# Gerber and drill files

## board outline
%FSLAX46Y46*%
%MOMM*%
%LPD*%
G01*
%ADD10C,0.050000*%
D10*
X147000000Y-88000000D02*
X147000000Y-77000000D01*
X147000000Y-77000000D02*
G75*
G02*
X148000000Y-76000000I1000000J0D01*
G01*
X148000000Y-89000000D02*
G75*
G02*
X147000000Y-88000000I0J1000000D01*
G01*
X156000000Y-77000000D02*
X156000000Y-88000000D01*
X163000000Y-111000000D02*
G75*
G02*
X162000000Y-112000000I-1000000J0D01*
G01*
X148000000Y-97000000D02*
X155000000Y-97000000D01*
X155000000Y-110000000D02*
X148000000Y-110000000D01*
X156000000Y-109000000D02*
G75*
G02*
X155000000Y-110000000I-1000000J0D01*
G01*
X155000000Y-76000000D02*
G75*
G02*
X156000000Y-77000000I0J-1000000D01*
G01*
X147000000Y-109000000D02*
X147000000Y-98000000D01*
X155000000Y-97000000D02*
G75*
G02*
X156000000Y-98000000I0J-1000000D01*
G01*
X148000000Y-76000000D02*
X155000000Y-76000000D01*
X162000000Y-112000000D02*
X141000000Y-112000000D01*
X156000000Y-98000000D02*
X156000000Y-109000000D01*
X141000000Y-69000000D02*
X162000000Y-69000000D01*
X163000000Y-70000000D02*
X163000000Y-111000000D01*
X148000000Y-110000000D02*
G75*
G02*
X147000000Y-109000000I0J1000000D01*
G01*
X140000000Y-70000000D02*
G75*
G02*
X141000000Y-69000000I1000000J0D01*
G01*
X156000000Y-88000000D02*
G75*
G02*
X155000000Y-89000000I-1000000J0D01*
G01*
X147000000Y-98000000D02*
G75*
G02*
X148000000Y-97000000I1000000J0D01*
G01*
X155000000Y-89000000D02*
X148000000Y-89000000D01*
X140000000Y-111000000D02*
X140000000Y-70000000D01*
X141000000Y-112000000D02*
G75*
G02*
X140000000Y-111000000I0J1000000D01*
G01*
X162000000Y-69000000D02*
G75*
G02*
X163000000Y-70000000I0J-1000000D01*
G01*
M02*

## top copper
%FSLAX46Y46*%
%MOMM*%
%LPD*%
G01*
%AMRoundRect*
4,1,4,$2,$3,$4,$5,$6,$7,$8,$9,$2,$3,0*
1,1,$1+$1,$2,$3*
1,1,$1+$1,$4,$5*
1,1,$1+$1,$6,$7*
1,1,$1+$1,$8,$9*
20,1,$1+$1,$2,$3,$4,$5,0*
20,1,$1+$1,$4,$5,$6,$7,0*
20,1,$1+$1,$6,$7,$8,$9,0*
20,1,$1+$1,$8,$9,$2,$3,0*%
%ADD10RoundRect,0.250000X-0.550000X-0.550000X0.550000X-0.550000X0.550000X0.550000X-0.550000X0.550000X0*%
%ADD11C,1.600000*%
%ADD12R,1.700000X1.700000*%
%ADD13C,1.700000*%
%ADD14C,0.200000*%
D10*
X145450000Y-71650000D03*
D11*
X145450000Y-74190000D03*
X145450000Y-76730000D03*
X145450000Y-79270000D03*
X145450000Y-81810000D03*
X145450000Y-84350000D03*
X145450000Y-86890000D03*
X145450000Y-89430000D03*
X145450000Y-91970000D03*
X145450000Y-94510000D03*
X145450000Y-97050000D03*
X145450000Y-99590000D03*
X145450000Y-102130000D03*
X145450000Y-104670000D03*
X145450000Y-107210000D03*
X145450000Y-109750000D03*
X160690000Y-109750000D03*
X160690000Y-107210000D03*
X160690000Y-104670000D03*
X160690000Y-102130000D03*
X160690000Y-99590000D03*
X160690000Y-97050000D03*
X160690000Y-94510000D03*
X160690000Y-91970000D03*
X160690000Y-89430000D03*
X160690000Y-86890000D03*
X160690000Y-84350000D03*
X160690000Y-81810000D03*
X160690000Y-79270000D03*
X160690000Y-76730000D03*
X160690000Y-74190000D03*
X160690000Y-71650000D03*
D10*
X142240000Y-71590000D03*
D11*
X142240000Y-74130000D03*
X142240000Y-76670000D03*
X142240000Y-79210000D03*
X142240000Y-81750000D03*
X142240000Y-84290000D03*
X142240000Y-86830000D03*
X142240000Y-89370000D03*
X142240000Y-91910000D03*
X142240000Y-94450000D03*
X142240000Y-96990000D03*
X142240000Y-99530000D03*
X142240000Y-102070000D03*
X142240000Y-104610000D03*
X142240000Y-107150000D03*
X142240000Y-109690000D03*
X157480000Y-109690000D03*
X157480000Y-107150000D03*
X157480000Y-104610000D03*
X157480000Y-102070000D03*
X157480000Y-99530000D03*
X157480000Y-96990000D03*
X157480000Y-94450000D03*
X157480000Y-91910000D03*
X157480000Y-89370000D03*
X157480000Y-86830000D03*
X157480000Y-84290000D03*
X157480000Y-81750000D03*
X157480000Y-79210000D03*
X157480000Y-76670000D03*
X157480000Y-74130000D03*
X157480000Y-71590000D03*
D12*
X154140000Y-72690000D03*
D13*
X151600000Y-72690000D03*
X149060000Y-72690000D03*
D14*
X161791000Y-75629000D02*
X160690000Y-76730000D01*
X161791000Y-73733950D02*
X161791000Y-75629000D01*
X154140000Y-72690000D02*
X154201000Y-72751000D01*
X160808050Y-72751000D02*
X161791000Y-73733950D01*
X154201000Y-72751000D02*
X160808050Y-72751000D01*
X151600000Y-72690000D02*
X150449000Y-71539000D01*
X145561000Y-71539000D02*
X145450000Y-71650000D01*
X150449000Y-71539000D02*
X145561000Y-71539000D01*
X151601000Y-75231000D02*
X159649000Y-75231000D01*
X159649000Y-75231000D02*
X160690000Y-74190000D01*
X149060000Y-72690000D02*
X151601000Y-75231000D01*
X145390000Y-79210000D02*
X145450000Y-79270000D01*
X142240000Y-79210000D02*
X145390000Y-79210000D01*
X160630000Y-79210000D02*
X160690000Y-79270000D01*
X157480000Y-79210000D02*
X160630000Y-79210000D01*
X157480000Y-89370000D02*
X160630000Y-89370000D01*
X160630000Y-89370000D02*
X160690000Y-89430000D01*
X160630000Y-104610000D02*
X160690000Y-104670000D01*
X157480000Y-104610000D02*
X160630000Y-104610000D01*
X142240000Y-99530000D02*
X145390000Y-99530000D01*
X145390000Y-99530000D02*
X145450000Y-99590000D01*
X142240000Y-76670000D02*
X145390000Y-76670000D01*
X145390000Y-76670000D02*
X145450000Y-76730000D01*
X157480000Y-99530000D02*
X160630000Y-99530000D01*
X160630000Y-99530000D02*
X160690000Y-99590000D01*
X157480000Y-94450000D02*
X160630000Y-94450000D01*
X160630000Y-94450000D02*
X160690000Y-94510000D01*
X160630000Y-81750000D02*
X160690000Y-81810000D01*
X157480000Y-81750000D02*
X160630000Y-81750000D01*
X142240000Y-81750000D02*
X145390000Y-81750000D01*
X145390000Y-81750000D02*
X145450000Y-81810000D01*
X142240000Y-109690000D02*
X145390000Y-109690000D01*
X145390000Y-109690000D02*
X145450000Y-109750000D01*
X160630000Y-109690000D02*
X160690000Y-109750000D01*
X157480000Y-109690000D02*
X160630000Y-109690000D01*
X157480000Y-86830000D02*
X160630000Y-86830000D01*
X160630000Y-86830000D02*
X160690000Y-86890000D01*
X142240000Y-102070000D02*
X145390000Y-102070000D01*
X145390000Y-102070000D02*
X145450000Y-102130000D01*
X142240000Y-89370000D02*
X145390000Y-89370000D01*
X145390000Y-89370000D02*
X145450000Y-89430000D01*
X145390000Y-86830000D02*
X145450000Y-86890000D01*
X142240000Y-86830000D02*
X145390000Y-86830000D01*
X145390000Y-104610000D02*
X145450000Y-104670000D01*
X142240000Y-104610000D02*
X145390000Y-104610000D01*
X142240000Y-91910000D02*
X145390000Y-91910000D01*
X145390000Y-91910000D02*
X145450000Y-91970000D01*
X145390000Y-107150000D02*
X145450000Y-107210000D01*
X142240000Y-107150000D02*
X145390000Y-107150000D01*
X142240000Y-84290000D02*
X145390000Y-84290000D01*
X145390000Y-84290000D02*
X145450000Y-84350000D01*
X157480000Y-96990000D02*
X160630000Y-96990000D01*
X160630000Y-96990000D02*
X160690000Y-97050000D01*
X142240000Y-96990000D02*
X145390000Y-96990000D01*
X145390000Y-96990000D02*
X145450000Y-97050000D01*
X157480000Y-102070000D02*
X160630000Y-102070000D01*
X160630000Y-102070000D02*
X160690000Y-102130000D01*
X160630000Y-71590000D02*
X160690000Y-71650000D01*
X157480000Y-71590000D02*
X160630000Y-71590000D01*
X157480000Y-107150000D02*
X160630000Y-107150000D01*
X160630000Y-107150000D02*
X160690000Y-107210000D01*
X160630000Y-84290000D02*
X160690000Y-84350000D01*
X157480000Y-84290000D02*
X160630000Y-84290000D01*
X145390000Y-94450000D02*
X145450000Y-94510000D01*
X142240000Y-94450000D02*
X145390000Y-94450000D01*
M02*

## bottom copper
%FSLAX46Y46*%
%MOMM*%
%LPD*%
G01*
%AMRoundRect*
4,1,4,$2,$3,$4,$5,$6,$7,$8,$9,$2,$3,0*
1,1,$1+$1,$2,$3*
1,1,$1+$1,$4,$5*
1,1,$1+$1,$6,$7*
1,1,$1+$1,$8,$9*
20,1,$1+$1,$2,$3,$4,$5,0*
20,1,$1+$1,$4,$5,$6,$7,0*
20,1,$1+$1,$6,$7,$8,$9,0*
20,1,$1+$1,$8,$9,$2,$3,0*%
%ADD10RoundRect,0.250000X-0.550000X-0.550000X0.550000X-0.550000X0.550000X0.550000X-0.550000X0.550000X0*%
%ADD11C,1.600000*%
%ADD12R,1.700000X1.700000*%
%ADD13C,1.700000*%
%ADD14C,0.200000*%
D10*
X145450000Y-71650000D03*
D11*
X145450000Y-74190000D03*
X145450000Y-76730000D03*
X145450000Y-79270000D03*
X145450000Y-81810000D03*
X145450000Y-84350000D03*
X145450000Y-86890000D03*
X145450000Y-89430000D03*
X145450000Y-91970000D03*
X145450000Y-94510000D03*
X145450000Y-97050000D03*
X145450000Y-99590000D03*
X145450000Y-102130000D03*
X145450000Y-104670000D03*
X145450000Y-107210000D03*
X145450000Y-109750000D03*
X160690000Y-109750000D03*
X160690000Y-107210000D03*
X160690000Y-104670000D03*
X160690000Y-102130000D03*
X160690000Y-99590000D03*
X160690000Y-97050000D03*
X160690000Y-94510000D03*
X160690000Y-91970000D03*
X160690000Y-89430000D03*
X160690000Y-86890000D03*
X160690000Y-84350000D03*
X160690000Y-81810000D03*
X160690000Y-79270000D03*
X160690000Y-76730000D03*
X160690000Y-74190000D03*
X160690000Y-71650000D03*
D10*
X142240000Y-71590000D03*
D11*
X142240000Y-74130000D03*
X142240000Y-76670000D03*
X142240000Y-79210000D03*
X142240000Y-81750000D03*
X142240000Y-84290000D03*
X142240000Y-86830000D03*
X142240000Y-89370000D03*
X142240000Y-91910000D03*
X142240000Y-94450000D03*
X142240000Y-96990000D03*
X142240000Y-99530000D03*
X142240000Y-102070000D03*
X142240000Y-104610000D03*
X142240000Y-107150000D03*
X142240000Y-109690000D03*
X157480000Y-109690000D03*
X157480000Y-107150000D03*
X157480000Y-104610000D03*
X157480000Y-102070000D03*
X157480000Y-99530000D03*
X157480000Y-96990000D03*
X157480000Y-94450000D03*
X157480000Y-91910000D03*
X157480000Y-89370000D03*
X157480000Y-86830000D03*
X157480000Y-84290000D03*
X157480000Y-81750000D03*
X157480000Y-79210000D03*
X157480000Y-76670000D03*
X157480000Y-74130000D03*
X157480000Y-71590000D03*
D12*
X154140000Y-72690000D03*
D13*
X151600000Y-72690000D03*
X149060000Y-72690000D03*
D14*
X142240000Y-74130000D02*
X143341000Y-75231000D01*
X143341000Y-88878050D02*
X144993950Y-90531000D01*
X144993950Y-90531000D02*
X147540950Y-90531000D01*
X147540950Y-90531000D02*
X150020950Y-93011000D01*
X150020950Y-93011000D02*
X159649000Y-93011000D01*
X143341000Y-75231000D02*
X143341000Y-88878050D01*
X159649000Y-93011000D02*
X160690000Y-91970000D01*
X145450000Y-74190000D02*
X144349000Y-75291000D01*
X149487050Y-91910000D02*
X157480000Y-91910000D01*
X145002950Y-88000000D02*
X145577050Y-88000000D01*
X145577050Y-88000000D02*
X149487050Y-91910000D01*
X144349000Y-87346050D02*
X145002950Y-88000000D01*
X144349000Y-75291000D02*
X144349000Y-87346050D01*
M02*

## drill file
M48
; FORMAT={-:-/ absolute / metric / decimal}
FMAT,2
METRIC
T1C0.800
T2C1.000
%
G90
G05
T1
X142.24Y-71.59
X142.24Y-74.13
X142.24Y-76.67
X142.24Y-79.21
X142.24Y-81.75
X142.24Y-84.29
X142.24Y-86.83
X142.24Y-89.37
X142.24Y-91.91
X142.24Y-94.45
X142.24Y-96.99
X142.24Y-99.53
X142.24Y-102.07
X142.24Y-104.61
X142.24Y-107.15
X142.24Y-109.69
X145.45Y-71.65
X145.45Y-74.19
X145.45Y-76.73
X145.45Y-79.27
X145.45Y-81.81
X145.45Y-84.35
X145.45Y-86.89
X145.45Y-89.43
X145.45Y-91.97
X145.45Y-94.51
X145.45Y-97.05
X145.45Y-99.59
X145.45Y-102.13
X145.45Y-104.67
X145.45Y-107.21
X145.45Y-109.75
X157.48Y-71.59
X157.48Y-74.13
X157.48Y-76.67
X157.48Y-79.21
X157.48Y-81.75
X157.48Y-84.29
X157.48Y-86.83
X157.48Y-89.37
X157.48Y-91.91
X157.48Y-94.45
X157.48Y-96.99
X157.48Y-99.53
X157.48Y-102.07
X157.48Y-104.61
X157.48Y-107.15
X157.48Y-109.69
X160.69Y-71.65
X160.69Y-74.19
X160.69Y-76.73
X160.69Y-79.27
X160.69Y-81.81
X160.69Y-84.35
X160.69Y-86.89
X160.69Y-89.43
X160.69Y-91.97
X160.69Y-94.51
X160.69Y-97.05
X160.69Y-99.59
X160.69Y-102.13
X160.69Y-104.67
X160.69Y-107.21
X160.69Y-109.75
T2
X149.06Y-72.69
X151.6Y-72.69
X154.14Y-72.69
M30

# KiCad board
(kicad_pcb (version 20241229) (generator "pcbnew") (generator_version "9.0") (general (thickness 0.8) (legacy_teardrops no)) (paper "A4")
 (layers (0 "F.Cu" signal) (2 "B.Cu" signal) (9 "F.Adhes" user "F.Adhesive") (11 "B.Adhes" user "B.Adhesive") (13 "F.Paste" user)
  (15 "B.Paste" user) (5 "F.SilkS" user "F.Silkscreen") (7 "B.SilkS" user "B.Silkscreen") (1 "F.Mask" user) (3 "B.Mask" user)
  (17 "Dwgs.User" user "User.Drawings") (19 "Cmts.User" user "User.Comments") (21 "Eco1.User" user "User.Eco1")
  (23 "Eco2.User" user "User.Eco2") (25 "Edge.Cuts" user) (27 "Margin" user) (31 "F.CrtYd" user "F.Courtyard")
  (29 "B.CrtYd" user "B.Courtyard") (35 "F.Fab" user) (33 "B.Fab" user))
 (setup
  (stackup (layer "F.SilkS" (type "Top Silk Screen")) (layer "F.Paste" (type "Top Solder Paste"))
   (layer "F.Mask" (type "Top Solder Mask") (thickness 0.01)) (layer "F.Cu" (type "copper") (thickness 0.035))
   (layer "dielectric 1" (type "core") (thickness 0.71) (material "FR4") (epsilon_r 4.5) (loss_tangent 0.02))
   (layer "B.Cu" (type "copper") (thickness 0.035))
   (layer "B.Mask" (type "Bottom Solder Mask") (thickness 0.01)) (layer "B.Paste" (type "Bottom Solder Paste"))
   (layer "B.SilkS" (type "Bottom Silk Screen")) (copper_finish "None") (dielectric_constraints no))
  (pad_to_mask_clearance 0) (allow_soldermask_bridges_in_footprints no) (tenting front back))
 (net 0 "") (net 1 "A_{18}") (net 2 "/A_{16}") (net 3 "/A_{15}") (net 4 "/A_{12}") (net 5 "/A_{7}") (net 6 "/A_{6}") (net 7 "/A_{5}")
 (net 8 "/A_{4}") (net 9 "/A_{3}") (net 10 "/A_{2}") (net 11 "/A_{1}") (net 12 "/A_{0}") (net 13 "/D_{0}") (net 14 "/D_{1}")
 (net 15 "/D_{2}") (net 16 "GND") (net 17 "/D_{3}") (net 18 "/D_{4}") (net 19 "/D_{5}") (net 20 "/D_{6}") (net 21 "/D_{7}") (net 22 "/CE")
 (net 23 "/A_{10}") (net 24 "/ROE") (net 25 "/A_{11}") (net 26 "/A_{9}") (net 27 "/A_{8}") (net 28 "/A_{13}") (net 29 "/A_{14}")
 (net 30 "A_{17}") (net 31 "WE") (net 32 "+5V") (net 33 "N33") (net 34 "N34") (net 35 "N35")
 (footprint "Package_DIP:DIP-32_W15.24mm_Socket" (layer "F.Cu") (at 145.45 71.65)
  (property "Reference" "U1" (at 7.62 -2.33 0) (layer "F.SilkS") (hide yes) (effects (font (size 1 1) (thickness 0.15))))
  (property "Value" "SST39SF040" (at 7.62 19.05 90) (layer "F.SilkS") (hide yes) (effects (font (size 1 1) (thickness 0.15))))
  (pad "1" thru_hole roundrect (at 0 0) (size 1.6 1.6) (drill 0.8) (layers "*.Cu" "*.Mask") (remove_unused_layers no)
   (roundrect_rratio 0.15625) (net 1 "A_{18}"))
  (pad "2" thru_hole circle (at 0 2.54) (size 1.6 1.6) (drill 0.8) (layers "*.Cu" "*.Mask") (remove_unused_layers no) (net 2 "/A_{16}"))
  (pad "3" thru_hole circle (at 0 5.08) (size 1.6 1.6) (drill 0.8) (layers "*.Cu" "*.Mask") (remove_unused_layers no) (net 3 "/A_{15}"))
  (pad "4" thru_hole circle (at 0 7.62) (size 1.6 1.6) (drill 0.8) (layers "*.Cu" "*.Mask") (remove_unused_layers no) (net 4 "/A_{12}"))
  (pad "5" thru_hole circle (at 0 10.16) (size 1.6 1.6) (drill 0.8) (layers "*.Cu" "*.Mask") (remove_unused_layers no) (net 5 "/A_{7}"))
  (pad "6" thru_hole circle (at 0 12.7) (size 1.6 1.6) (drill 0.8) (layers "*.Cu" "*.Mask") (remove_unused_layers no) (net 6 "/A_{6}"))
  (pad "7" thru_hole circle (at 0 15.24) (size 1.6 1.6) (drill 0.8) (layers "*.Cu" "*.Mask") (remove_unused_layers no) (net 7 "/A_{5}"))
  (pad "8" thru_hole circle (at 0 17.78) (size 1.6 1.6) (drill 0.8) (layers "*.Cu" "*.Mask") (remove_unused_layers no) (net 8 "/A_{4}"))
  (pad "9" thru_hole circle (at 0 20.32) (size 1.6 1.6) (drill 0.8) (layers "*.Cu" "*.Mask") (remove_unused_layers no) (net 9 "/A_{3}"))
  (pad "10" thru_hole circle (at 0 22.86) (size 1.6 1.6) (drill 0.8) (layers "*.Cu" "*.Mask") (remove_unused_layers no) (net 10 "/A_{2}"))
  (pad "11" thru_hole circle (at 0 25.4) (size 1.6 1.6) (drill 0.8) (layers "*.Cu" "*.Mask") (remove_unused_layers no) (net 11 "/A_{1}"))
  (pad "12" thru_hole circle (at 0 27.94) (size 1.6 1.6) (drill 0.8) (layers "*.Cu" "*.Mask") (remove_unused_layers no) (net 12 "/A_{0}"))
  (pad "13" thru_hole circle (at 0 30.48) (size 1.6 1.6) (drill 0.8) (layers "*.Cu" "*.Mask") (remove_unused_layers no) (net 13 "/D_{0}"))
  (pad "14" thru_hole circle (at 0 33.02) (size 1.6 1.6) (drill 0.8) (layers "*.Cu" "*.Mask") (remove_unused_layers no) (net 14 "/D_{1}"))
  (pad "15" thru_hole circle (at 0 35.56) (size 1.6 1.6) (drill 0.8) (layers "*.Cu" "*.Mask") (remove_unused_layers no) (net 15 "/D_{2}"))
  (pad "16" thru_hole circle (at 0 38.1) (size 1.6 1.6) (drill 0.8) (layers "*.Cu" "*.Mask") (remove_unused_layers no) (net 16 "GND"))
  (pad "17" thru_hole circle (at 15.24 38.1) (size 1.6 1.6) (drill 0.8) (layers "*.Cu" "*.Mask") (remove_unused_layers no) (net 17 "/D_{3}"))
  (pad "18" thru_hole circle (at 15.24 35.56) (size 1.6 1.6) (drill 0.8) (layers "*.Cu" "*.Mask") (remove_unused_layers no)
   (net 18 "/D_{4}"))
  (pad "19" thru_hole circle (at 15.24 33.02) (size 1.6 1.6) (drill 0.8) (layers "*.Cu" "*.Mask") (remove_unused_layers no)
   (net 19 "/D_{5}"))
  (pad "20" thru_hole circle (at 15.24 30.48) (size 1.6 1.6) (drill 0.8) (layers "*.Cu" "*.Mask") (remove_unused_layers no)
   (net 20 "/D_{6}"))
  (pad "21" thru_hole circle (at 15.24 27.94) (size 1.6 1.6) (drill 0.8) (layers "*.Cu" "*.Mask") (remove_unused_layers no)
   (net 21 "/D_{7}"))
  (pad "22" thru_hole circle (at 15.24 25.4) (size 1.6 1.6) (drill 0.8) (layers "*.Cu" "*.Mask") (remove_unused_layers no) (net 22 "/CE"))
  (pad "23" thru_hole circle (at 15.24 22.86) (size 1.6 1.6) (drill 0.8) (layers "*.Cu" "*.Mask") (remove_unused_layers no)
   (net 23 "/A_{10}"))
  (pad "24" thru_hole circle (at 15.24 20.32) (size 1.6 1.6) (drill 0.8) (layers "*.Cu" "*.Mask") (remove_unused_layers no) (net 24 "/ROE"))
  (pad "25" thru_hole circle (at 15.24 17.78) (size 1.6 1.6) (drill 0.8) (layers "*.Cu" "*.Mask") (remove_unused_layers no)
   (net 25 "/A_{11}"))
  (pad "26" thru_hole circle (at 15.24 15.24) (size 1.6 1.6) (drill 0.8) (layers "*.Cu" "*.Mask") (remove_unused_layers no)
   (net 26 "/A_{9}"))
  (pad "27" thru_hole circle (at 15.24 12.7) (size 1.6 1.6) (drill 0.8) (layers "*.Cu" "*.Mask") (remove_unused_layers no) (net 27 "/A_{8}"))
  (pad "28" thru_hole circle (at 15.24 10.16) (size 1.6 1.6) (drill 0.8) (layers "*.Cu" "*.Mask") (remove_unused_layers no)
   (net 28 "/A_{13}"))
  (pad "29" thru_hole circle (at 15.24 7.62) (size 1.6 1.6) (drill 0.8) (layers "*.Cu" "*.Mask") (remove_unused_layers no)
   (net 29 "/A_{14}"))
  (pad "30" thru_hole circle (at 15.24 5.08) (size 1.6 1.6) (drill 0.8) (layers "*.Cu" "*.Mask") (remove_unused_layers no) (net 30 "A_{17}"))
  (pad "31" thru_hole circle (at 15.24 2.54) (size 1.6 1.6) (drill 0.8) (layers "*.Cu" "*.Mask") (remove_unused_layers no) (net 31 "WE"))
  (pad "32" thru_hole circle (at 15.24 0) (size 1.6 1.6) (drill 0.8) (layers "*.Cu" "*.Mask") (remove_unused_layers no) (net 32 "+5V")))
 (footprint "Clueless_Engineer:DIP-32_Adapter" (layer "F.Cu") (at 142.32 71.53)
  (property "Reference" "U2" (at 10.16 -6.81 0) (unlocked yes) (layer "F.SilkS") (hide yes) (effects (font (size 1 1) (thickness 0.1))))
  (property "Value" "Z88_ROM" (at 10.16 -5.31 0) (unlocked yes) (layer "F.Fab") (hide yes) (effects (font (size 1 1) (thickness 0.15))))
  (pad "1" thru_hole roundrect (at -0.08 0.06) (size 1.6 1.6) (drill 0.8) (layers "*.Cu" "*.Mask") (remove_unused_layers no)
   (roundrect_rratio 0.15625) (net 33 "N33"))
  (pad "2" thru_hole circle (at -0.08 2.6) (size 1.6 1.6) (drill 0.8) (layers "*.Cu" "*.Mask") (remove_unused_layers no) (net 24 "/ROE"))
  (pad "3" thru_hole circle (at -0.08 5.14) (size 1.6 1.6) (drill 0.8) (layers "*.Cu" "*.Mask") (remove_unused_layers no) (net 3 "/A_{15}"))
  (pad "4" thru_hole circle (at -0.08 7.68) (size 1.6 1.6) (drill 0.8) (layers "*.Cu" "*.Mask") (remove_unused_layers no) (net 4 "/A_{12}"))
  (pad "5" thru_hole circle (at -0.08 10.22) (size 1.6 1.6) (drill 0.8) (layers "*.Cu" "*.Mask") (remove_unused_layers no) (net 5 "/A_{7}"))
  (pad "6" thru_hole circle (at -0.08 12.76) (size 1.6 1.6) (drill 0.8) (layers "*.Cu" "*.Mask") (remove_unused_layers no) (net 6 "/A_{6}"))
  (pad "7" thru_hole circle (at -0.08 15.3) (size 1.6 1.6) (drill 0.8) (layers "*.Cu" "*.Mask") (remove_unused_layers no) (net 7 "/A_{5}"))
  (pad "8" thru_hole circle (at -0.08 17.84) (size 1.6 1.6) (drill 0.8) (layers "*.Cu" "*.Mask") (remove_unused_layers no) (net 8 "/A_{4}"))
  (pad "9" thru_hole circle (at -0.08 20.38) (size 1.6 1.6) (drill 0.8) (layers "*.Cu" "*.Mask") (remove_unused_layers no) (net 9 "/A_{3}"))
  (pad "10" thru_hole circle (at -0.08 22.92) (size 1.6 1.6) (drill 0.8) (layers "*.Cu" "*.Mask") (remove_unused_layers no)
   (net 10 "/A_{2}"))
  (pad "11" thru_hole circle (at -0.08 25.46) (size 1.6 1.6) (drill 0.8) (layers "*.Cu" "*.Mask") (remove_unused_layers no)
   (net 11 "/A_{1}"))
  (pad "12" thru_hole circle (at -0.08 28) (size 1.6 1.6) (drill 0.8) (layers "*.Cu" "*.Mask") (remove_unused_layers no) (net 12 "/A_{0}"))
  (pad "13" thru_hole circle (at -0.08 30.54) (size 1.6 1.6) (drill 0.8) (layers "*.Cu" "*.Mask") (remove_unused_layers no)
   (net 13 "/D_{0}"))
  (pad "14" thru_hole circle (at -0.08 33.08) (size 1.6 1.6) (drill 0.8) (layers "*.Cu" "*.Mask") (remove_unused_layers no)
   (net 14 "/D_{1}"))
  (pad "15" thru_hole circle (at -0.08 35.62) (size 1.6 1.6) (drill 0.8) (layers "*.Cu" "*.Mask") (remove_unused_layers no)
   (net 15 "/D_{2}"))
  (pad "16" thru_hole circle (at -0.08 38.16) (size 1.6 1.6) (drill 0.8) (layers "*.Cu" "*.Mask") (remove_unused_layers no) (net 16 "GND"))
  (pad "17" thru_hole circle (at 15.16 38.16) (size 1.6 1.6) (drill 0.8) (layers "*.Cu" "*.Mask") (remove_unused_layers no)
   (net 17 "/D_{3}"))
  (pad "18" thru_hole circle (at 15.16 35.62) (size 1.6 1.6) (drill 0.8) (layers "*.Cu" "*.Mask") (remove_unused_layers no)
   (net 18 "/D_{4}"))
  (pad "19" thru_hole circle (at 15.16 33.08) (size 1.6 1.6) (drill 0.8) (layers "*.Cu" "*.Mask") (remove_unused_layers no)
   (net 19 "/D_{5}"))
  (pad "20" thru_hole circle (at 15.16 30.54) (size 1.6 1.6) (drill 0.8) (layers "*.Cu" "*.Mask") (remove_unused_layers no)
   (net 20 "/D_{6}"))
  (pad "21" thru_hole circle (at 15.16 28) (size 1.6 1.6) (drill 0.8) (layers "*.Cu" "*.Mask") (remove_unused_layers no) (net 21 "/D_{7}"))
  (pad "22" thru_hole circle (at 15.16 25.46) (size 1.6 1.6) (drill 0.8) (layers "*.Cu" "*.Mask") (remove_unused_layers no) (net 22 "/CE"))
  (pad "23" thru_hole circle (at 15.16 22.92) (size 1.6 1.6) (drill 0.8) (layers "*.Cu" "*.Mask") (remove_unused_layers no)
   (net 23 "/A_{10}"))
  (pad "24" thru_hole circle (at 15.16 20.38) (size 1.6 1.6) (drill 0.8) (layers "*.Cu" "*.Mask") (remove_unused_layers no)
   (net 2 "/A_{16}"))
  (pad "25" thru_hole circle (at 15.16 17.84) (size 1.6 1.6) (drill 0.8) (layers "*.Cu" "*.Mask") (remove_unused_layers no)
   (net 25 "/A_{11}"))
  (pad "26" thru_hole circle (at 15.16 15.3) (size 1.6 1.6) (drill 0.8) (layers "*.Cu" "*.Mask") (remove_unused_layers no) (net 26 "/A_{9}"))
  (pad "27" thru_hole circle (at 15.16 12.76) (size 1.6 1.6) (drill 0.8) (layers "*.Cu" "*.Mask") (remove_unused_layers no)
   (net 27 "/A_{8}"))
  (pad "28" thru_hole circle (at 15.16 10.22) (size 1.6 1.6) (drill 0.8) (layers "*.Cu" "*.Mask") (remove_unused_layers no)
   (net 28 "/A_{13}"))
  (pad "29" thru_hole circle (at 15.16 7.68) (size 1.6 1.6) (drill 0.8) (layers "*.Cu" "*.Mask") (remove_unused_layers no)
   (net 29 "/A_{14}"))
  (pad "30" thru_hole circle (at 15.16 5.14) (size 1.6 1.6) (drill 0.8) (layers "*.Cu" "*.Mask") (remove_unused_layers no) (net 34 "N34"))
  (pad "31" thru_hole circle (at 15.16 2.6) (size 1.6 1.6) (drill 0.8) (layers "*.Cu" "*.Mask") (remove_unused_layers no) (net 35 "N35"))
  (pad "32" thru_hole circle (at 15.16 0.06) (size 1.6 1.6) (drill 0.8) (layers "*.Cu" "*.Mask") (remove_unused_layers no) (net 32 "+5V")))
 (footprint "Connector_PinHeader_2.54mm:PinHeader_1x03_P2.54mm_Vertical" (layer "F.Cu") (at 154.14 72.69 -90)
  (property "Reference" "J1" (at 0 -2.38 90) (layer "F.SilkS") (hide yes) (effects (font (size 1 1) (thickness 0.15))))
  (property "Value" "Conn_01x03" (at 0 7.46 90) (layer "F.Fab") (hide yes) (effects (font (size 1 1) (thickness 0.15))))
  (pad "1" thru_hole rect (at 0 0 270) (size 1.7 1.7) (drill 1) (layers "*.Cu" "*.Mask") (remove_unused_layers no) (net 30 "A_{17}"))
  (pad "2" thru_hole circle (at 0 2.54 270) (size 1.7 1.7) (drill 1) (layers "*.Cu" "*.Mask") (remove_unused_layers no) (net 1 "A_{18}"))
  (pad "3" thru_hole circle (at 0 5.08 270) (size 1.7 1.7) (drill 1) (layers "*.Cu" "*.Mask") (remove_unused_layers no) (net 31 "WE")))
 (gr_line (start 147 88) (end 147 77) (stroke (width 0.05) (type default)) (layer "Edge.Cuts"))
 (gr_arc (start 147 77) (mid 147.292893 76.292893) (end 148 76) (stroke (width 0.05) (type default)) (layer "Edge.Cuts"))
 (gr_arc (start 148 89) (mid 147.292893 88.707107) (end 147 88) (stroke (width 0.05) (type default)) (layer "Edge.Cuts"))
 (gr_line (start 156 77) (end 156 88) (stroke (width 0.05) (type default)) (layer "Edge.Cuts"))
 (gr_arc (start 163 111) (mid 162.707107 111.707107) (end 162 112) (stroke (width 0.05) (type default)) (layer "Edge.Cuts"))
 (gr_line (start 148 97) (end 155 97) (stroke (width 0.05) (type default)) (layer "Edge.Cuts"))
 (gr_line (start 155 110) (end 148 110) (stroke (width 0.05) (type default)) (layer "Edge.Cuts"))
 (gr_arc (start 156 109) (mid 155.707107 109.707107) (end 155 110) (stroke (width 0.05) (type default)) (layer "Edge.Cuts"))
 (gr_arc (start 155 76) (mid 155.707107 76.292893) (end 156 77) (stroke (width 0.05) (type default)) (layer "Edge.Cuts"))
 (gr_line (start 147 109) (end 147 98) (stroke (width 0.05) (type default)) (layer "Edge.Cuts"))
 (gr_arc (start 155 97) (mid 155.707107 97.292893) (end 156 98) (stroke (width 0.05) (type default)) (layer "Edge.Cuts"))
 (gr_line (start 148 76) (end 155 76) (stroke (width 0.05) (type default)) (layer "Edge.Cuts"))
 (gr_line (start 162 112) (end 141 112) (stroke (width 0.05) (type default)) (layer "Edge.Cuts"))
 (gr_line (start 156 98) (end 156 109) (stroke (width 0.05) (type default)) (layer "Edge.Cuts"))
 (gr_line (start 141 69) (end 162 69) (stroke (width 0.05) (type default)) (layer "Edge.Cuts"))
 (gr_line (start 163 70) (end 163 111) (stroke (width 0.05) (type default)) (layer "Edge.Cuts"))
 (gr_arc (start 148 110) (mid 147.292893 109.707107) (end 147 109) (stroke (width 0.05) (type default)) (layer "Edge.Cuts"))
 (gr_arc (start 140 70) (mid 140.292893 69.292893) (end 141 69) (stroke (width 0.05) (type default)) (layer "Edge.Cuts"))
 (gr_arc (start 156 88) (mid 155.707107 88.707107) (end 155 89) (stroke (width 0.05) (type default)) (layer "Edge.Cuts"))
 (gr_arc (start 147 98) (mid 147.292893 97.292893) (end 148 97) (stroke (width 0.05) (type default)) (layer "Edge.Cuts"))
 (gr_line (start 155 89) (end 148 89) (stroke (width 0.05) (type default)) (layer "Edge.Cuts"))
 (gr_line (start 140 111) (end 140 70) (stroke (width 0.05) (type default)) (layer "Edge.Cuts"))
 (gr_arc (start 141 112) (mid 140.292893 111.707107) (end 140 111) (stroke (width 0.05) (type default)) (layer "Edge.Cuts"))
 (gr_arc (start 162 69) (mid 162.707107 69.292893) (end 163 70) (stroke (width 0.05) (type default)) (layer "Edge.Cuts"))
 (segment (start 161.791 75.629) (end 160.69 76.73) (width 0.2) (layer "F.Cu") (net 30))
 (segment (start 161.791 73.73395) (end 161.791 75.629) (width 0.2) (layer "F.Cu") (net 30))
 (segment (start 154.14 72.69) (end 154.201 72.751) (width 0.2) (layer "F.Cu") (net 30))
 (segment (start 160.80805 72.751) (end 161.791 73.73395) (width 0.2) (layer "F.Cu") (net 30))
 (segment (start 154.201 72.751) (end 160.80805 72.751) (width 0.2) (layer "F.Cu") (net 30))
 (segment (start 151.6 72.69) (end 150.449 71.539) (width 0.2) (layer "F.Cu") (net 1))
 (segment (start 145.561 71.539) (end 145.45 71.65) (width 0.2) (layer "F.Cu") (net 1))
 (segment (start 150.449 71.539) (end 145.561 71.539) (width 0.2) (layer "F.Cu") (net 1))
 (segment (start 151.601 75.231) (end 159.649 75.231) (width 0.2) (layer "F.Cu") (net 31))
 (segment (start 159.649 75.231) (end 160.69 74.19) (width 0.2) (layer "F.Cu") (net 31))
 (segment (start 149.06 72.69) (end 151.601 75.231) (width 0.2) (layer "F.Cu") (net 31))
 (segment (start 145.39 79.21) (end 145.45 79.27) (width 0.2) (layer "F.Cu") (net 4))
 (segment (start 142.24 79.21) (end 145.39 79.21) (width 0.2) (layer "F.Cu") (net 4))
 (segment (start 160.63 79.21) (end 160.69 79.27) (width 0.2) (layer "F.Cu") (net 29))
 (segment (start 157.48 79.21) (end 160.63 79.21) (width 0.2) (layer "F.Cu") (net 29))
 (segment (start 157.48 89.37) (end 160.63 89.37) (width 0.2) (layer "F.Cu") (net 25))
 (segment (start 160.63 89.37) (end 160.69 89.43) (width 0.2) (layer "F.Cu") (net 25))
 (segment (start 160.63 104.61) (end 160.69 104.67) (width 0.2) (layer "F.Cu") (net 19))
 (segment (start 157.48 104.61) (end 160.63 104.61) (width 0.2) (layer "F.Cu") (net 19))
 (segment (start 142.24 99.53) (end 145.39 99.53) (width 0.2) (layer "F.Cu") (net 12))
 (segment (start 145.39 99.53) (end 145.45 99.59) (width 0.2) (layer "F.Cu") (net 12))
 (segment (start 142.24 76.67) (end 145.39 76.67) (width 0.2) (layer "F.Cu") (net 3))
 (segment (start 145.39 76.67) (end 145.45 76.73) (width 0.2) (layer "F.Cu") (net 3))
 (segment (start 157.48 99.53) (end 160.63 99.53) (width 0.2) (layer "F.Cu") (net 21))
 (segment (start 160.63 99.53) (end 160.69 99.59) (width 0.2) (layer "F.Cu") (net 21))
 (segment (start 157.48 94.45) (end 160.63 94.45) (width 0.2) (layer "F.Cu") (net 23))
 (segment (start 160.63 94.45) (end 160.69 94.51) (width 0.2) (layer "F.Cu") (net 23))
 (segment (start 160.63 81.75) (end 160.69 81.81) (width 0.2) (layer "F.Cu") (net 28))
 (segment (start 157.48 81.75) (end 160.63 81.75) (width 0.2) (layer "F.Cu") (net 28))
 (segment (start 142.24 81.75) (end 145.39 81.75) (width 0.2) (layer "F.Cu") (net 5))
 (segment (start 145.39 81.75) (end 145.45 81.81) (width 0.2) (layer "F.Cu") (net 5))
 (segment (start 142.24 109.69) (end 145.39 109.69) (width 0.2) (layer "F.Cu") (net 16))
 (segment (start 145.39 109.69) (end 145.45 109.75) (width 0.2) (layer "F.Cu") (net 16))
 (segment (start 160.63 109.69) (end 160.69 109.75) (width 0.2) (layer "F.Cu") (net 17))
 (segment (start 157.48 109.69) (end 160.63 109.69) (width 0.2) (layer "F.Cu") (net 17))
 (segment (start 157.48 86.83) (end 160.63 86.83) (width 0.2) (layer "F.Cu") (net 26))
 (segment (start 160.63 86.83) (end 160.69 86.89) (width 0.2) (layer "F.Cu") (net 26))
 (segment (start 142.24 102.07) (end 145.39 102.07) (width 0.2) (layer "F.Cu") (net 13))
 (segment (start 145.39 102.07) (end 145.45 102.13) (width 0.2) (layer "F.Cu") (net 13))
 (segment (start 142.24 89.37) (end 145.39 89.37) (width 0.2) (layer "F.Cu") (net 8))
 (segment (start 145.39 89.37) (end 145.45 89.43) (width 0.2) (layer "F.Cu") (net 8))
 (segment (start 145.39 86.83) (end 145.45 86.89) (width 0.2) (layer "F.Cu") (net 7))
 (segment (start 142.24 86.83) (end 145.39 86.83) (width 0.2) (layer "F.Cu") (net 7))
 (segment (start 142.24 74.13) (end 143.341 75.231) (width 0.2) (layer "B.Cu") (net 24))
 (segment (start 143.341 88.87805) (end 144.99395 90.531) (width 0.2) (layer "B.Cu") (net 24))
 (segment (start 144.99395 90.531) (end 147.54095 90.531) (width 0.2) (layer "B.Cu") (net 24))
 (segment (start 147.54095 90.531) (end 150.02095 93.011) (width 0.2) (layer "B.Cu") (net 24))
 (segment (start 150.02095 93.011) (end 159.649 93.011) (width 0.2) (layer "B.Cu") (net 24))
 (segment (start 143.341 75.231) (end 143.341 88.87805) (width 0.2) (layer "B.Cu") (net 24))
 (segment (start 159.649 93.011) (end 160.69 91.97) (width 0.2) (layer "B.Cu") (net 24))
 (segment (start 145.39 104.61) (end 145.45 104.67) (width 0.2) (layer "F.Cu") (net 14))
 (segment (start 142.24 104.61) (end 145.39 104.61) (width 0.2) (layer "F.Cu") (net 14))
 (segment (start 142.24 91.91) (end 145.39 91.91) (width 0.2) (layer "F.Cu") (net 9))
 (segment (start 145.39 91.91) (end 145.45 91.97) (width 0.2) (layer "F.Cu") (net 9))
 (segment (start 145.39 107.15) (end 145.45 107.21) (width 0.2) (layer "F.Cu") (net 15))
 (segment (start 142.24 107.15) (end 145.39 107.15) (width 0.2) (layer "F.Cu") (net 15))
 (segment (start 145.45 74.19) (end 144.349 75.291) (width 0.2) (layer "B.Cu") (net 2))
 (segment (start 149.48705 91.91) (end 157.48 91.91) (width 0.2) (layer "B.Cu") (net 2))
 (segment (start 145.00295 88) (end 145.57705 88) (width 0.2) (layer "B.Cu") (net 2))
 (segment (start 145.57705 88) (end 149.48705 91.91) (width 0.2) (layer "B.Cu") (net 2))
 (segment (start 144.349 87.34605) (end 145.00295 88) (width 0.2) (layer "B.Cu") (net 2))
 (segment (start 144.349 75.291) (end 144.349 87.34605) (width 0.2) (layer "B.Cu") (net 2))
 (segment (start 142.24 84.29) (end 145.39 84.29) (width 0.2) (layer "F.Cu") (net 6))
 (segment (start 145.39 84.29) (end 145.45 84.35) (width 0.2) (layer "F.Cu") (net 6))
 (segment (start 157.48 96.99) (end 160.63 96.99) (width 0.2) (layer "F.Cu") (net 22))
 (segment (start 160.63 96.99) (end 160.69 97.05) (width 0.2) (layer "F.Cu") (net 22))
 (segment (start 142.24 96.99) (end 145.39 96.99) (width 0.2) (layer "F.Cu") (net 11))
 (segment (start 145.39 96.99) (end 145.45 97.05) (width 0.2) (layer "F.Cu") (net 11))
 (segment (start 157.48 102.07) (end 160.63 102.07) (width 0.2) (layer "F.Cu") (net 20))
 (segment (start 160.63 102.07) (end 160.69 102.13) (width 0.2) (layer "F.Cu") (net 20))
 (segment (start 160.63 71.59) (end 160.69 71.65) (width 0.2) (layer "F.Cu") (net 32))
 (segment (start 157.48 71.59) (end 160.63 71.59) (width 0.2) (layer "F.Cu") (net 32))
 (segment (start 157.48 107.15) (end 160.63 107.15) (width 0.2) (layer "F.Cu") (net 18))
 (segment (start 160.63 107.15) (end 160.69 107.21) (width 0.2) (layer "F.Cu") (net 18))
 (segment (start 160.63 84.29) (end 160.69 84.35) (width 0.2) (layer "F.Cu") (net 27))
 (segment (start 157.48 84.29) (end 160.63 84.29) (width 0.2) (layer "F.Cu") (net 27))
 (segment (start 145.39 94.45) (end 145.45 94.51) (width 0.2) (layer "F.Cu") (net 10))
 (segment (start 142.24 94.45) (end 145.39 94.45) (width 0.2) (layer "F.Cu") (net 10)))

